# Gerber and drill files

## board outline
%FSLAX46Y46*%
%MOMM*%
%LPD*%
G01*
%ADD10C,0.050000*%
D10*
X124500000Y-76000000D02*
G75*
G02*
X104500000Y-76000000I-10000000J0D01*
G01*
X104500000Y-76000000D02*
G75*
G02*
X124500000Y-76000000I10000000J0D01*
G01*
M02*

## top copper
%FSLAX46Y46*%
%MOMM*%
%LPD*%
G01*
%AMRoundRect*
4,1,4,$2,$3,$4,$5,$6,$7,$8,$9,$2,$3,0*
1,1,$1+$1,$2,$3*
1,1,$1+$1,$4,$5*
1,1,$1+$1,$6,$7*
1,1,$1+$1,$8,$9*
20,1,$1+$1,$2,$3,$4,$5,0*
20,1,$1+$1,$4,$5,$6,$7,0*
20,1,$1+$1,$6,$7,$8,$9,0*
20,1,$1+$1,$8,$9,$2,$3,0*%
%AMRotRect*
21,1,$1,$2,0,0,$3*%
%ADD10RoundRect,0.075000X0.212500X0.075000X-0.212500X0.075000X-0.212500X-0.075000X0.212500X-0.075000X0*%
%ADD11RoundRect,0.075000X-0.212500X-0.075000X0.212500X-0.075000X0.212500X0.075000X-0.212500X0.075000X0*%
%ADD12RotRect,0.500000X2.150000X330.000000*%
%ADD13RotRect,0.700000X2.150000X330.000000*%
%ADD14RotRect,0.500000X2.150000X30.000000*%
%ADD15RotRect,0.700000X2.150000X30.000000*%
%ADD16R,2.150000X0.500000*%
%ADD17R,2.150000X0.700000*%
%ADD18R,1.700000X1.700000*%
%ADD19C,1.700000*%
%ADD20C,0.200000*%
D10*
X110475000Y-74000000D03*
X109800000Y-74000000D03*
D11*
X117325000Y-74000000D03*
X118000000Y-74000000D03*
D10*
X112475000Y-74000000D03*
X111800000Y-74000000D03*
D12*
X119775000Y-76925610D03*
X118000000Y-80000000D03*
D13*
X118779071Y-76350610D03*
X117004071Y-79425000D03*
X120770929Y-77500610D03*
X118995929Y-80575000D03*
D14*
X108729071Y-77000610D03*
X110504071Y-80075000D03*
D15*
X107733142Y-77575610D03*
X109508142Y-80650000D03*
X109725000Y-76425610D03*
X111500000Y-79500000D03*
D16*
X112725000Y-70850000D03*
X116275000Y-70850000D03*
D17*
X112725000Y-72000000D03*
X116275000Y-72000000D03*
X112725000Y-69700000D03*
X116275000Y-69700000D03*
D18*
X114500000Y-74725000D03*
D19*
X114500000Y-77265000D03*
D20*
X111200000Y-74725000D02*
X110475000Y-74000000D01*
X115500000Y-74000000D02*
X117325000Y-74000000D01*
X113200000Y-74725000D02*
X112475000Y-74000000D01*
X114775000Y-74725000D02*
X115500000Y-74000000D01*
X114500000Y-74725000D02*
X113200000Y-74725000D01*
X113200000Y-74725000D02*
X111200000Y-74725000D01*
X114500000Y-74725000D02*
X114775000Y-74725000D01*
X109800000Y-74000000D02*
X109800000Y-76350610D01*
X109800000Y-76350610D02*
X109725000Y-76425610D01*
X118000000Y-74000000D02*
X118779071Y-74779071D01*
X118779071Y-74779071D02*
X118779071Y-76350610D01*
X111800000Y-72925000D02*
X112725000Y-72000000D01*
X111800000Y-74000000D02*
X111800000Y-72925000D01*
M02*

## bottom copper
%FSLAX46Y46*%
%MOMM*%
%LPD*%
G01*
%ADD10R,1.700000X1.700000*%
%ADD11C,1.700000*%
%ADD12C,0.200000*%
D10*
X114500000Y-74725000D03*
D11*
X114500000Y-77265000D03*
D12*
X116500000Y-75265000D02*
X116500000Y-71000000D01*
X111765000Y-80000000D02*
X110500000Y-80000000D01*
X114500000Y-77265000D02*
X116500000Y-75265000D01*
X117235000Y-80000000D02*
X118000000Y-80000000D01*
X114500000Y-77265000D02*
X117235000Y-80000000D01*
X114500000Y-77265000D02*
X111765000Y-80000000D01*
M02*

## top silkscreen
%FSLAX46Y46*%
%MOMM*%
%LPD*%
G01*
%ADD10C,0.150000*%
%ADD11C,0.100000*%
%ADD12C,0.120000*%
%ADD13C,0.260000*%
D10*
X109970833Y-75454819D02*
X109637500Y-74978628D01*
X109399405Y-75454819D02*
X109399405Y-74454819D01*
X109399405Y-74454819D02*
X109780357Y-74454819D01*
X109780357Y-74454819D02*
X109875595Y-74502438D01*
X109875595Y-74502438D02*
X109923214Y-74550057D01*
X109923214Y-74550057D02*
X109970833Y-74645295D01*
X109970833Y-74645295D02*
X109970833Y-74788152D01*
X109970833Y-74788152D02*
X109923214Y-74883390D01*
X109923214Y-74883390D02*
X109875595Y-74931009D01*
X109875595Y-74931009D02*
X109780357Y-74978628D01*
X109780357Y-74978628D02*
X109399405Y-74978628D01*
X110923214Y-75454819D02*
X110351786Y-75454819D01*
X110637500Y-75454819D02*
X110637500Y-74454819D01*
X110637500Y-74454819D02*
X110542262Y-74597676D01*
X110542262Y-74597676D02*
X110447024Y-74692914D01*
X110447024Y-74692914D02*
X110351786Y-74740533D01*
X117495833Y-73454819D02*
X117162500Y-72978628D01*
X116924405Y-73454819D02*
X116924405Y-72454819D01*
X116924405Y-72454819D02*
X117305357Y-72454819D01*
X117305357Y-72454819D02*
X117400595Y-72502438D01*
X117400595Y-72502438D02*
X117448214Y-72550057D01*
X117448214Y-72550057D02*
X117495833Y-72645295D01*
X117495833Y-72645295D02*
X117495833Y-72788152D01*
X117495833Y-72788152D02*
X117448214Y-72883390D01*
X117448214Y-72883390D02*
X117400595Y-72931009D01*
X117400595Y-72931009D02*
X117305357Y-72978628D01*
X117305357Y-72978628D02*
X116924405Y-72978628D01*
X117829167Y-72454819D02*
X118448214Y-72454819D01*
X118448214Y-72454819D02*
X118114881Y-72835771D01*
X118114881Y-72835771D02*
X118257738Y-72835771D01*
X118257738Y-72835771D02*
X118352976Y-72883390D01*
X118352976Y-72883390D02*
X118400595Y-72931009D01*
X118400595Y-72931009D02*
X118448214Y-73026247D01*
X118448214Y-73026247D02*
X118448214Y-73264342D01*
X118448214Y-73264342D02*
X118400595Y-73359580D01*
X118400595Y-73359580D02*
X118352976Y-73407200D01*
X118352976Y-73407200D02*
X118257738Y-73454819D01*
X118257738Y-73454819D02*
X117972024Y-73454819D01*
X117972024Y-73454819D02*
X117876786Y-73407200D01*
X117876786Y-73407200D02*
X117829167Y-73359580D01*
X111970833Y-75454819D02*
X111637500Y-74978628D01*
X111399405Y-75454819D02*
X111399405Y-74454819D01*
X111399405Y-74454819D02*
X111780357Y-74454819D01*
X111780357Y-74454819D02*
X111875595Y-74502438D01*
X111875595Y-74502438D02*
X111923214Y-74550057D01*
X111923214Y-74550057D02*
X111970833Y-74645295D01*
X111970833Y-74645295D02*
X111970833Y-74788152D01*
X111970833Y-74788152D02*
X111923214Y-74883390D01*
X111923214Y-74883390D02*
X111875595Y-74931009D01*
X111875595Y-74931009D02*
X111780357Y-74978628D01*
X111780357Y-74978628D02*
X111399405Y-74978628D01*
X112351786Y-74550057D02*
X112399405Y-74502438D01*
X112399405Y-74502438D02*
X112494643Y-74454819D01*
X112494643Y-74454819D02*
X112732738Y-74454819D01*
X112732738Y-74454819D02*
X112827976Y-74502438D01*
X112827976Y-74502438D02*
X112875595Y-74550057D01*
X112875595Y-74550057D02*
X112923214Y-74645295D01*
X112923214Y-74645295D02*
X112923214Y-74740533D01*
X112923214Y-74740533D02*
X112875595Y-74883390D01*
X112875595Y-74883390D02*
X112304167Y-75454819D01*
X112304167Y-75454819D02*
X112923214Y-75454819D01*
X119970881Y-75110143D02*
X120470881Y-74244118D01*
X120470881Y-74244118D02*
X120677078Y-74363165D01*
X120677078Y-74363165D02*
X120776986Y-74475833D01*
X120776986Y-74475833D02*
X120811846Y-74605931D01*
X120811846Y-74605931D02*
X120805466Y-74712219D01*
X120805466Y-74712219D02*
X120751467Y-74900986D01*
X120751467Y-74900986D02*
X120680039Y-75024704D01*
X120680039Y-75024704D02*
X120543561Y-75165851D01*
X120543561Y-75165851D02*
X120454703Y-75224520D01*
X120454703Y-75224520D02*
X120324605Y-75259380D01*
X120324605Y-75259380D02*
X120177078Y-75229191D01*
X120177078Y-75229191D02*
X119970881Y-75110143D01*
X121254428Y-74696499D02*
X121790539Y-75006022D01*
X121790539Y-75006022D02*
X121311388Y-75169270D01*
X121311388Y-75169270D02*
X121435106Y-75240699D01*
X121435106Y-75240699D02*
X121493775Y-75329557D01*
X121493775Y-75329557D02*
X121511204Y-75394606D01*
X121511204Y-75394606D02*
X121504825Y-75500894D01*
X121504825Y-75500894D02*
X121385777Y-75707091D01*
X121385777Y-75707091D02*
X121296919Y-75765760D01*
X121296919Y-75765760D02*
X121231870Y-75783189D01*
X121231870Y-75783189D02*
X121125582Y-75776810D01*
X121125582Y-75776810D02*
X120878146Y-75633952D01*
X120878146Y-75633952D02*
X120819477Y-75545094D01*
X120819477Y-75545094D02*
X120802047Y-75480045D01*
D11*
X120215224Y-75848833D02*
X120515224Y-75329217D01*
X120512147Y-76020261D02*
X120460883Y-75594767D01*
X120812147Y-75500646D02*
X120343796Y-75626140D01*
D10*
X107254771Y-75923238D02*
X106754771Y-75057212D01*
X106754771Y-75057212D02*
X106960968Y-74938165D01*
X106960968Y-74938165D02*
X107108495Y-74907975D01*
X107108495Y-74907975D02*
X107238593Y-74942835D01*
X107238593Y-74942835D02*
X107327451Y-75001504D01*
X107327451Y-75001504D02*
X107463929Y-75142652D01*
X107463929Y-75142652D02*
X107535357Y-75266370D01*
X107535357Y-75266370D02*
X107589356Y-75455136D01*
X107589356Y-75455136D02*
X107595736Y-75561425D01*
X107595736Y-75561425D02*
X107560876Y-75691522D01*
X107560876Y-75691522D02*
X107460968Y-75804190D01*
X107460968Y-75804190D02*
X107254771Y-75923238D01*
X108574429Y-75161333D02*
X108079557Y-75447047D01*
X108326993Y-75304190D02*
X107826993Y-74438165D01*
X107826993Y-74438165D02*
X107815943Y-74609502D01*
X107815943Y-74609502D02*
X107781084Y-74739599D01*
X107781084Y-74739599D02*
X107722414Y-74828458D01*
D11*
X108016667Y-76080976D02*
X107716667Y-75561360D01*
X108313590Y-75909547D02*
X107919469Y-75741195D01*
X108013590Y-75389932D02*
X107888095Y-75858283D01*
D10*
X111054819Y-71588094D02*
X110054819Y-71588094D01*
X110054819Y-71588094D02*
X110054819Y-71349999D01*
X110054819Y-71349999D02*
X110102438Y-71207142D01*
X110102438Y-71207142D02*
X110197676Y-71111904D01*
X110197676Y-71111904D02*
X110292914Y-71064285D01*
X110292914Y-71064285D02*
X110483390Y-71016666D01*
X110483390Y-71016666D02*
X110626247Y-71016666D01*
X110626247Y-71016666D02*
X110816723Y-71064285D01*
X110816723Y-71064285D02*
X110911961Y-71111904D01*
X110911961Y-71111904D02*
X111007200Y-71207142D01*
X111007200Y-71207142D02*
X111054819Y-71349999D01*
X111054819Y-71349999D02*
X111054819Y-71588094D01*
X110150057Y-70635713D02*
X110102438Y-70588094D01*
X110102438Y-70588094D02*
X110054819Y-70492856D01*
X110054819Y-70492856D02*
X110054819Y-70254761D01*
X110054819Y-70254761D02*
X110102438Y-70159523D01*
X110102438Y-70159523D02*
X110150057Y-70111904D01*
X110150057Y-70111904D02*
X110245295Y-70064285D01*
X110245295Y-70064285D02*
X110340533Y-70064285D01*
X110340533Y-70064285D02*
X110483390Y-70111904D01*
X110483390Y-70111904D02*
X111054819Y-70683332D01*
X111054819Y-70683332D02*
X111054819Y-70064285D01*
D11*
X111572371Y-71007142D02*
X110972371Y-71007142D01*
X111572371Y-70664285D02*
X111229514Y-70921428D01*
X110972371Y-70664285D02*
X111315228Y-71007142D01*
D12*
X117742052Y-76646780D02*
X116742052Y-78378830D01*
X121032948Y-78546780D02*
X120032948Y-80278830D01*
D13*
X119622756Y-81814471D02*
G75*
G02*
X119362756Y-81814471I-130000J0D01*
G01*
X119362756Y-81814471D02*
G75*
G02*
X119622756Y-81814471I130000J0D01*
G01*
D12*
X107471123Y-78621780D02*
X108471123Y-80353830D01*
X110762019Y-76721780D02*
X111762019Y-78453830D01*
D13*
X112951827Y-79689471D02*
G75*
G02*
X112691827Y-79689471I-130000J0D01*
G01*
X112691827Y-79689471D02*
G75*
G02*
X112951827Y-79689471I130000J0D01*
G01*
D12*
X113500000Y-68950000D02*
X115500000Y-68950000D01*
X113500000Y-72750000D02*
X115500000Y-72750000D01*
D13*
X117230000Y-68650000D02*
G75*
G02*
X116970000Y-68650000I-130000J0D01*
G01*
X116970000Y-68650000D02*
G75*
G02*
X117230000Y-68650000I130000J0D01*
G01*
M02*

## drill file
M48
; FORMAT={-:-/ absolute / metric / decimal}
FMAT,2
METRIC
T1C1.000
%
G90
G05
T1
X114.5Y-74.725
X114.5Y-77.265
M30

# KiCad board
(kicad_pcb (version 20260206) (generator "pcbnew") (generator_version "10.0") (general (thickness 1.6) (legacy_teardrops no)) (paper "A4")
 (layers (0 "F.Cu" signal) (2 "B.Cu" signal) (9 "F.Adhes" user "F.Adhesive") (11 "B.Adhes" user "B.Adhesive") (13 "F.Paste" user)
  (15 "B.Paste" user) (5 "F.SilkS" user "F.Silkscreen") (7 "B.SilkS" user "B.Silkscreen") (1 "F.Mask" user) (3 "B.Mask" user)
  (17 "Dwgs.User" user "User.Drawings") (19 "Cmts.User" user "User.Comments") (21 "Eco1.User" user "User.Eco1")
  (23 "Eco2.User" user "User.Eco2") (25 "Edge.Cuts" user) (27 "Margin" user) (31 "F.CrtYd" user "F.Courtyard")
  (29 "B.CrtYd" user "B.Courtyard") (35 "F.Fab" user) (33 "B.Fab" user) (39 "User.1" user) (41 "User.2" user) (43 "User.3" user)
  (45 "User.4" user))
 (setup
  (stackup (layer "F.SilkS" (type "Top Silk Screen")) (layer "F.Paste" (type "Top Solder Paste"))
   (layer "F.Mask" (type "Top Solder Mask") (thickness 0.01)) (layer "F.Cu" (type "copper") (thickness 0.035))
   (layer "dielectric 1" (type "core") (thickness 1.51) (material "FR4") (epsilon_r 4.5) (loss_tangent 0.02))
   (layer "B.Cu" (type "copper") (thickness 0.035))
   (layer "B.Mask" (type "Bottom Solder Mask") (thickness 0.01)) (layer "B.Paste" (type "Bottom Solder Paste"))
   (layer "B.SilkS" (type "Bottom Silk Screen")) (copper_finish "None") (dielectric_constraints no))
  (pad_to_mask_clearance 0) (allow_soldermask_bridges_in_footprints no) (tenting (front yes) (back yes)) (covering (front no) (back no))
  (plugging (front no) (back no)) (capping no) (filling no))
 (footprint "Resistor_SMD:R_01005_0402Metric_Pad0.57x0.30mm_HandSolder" (layer "F.Cu") (at 110.1375 74 180)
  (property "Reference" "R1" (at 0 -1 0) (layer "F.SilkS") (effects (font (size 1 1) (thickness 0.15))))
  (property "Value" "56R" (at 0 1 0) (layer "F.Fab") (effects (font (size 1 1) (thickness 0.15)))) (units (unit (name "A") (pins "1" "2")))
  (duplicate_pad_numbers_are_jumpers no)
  (pad "" smd roundrect (at -0.3625 0 180) (size 0.41 0.27) (layers "F.Paste") (roundrect_rratio 0.25))
  (pad "" smd roundrect (at 0.3625 0 180) (size 0.41 0.27) (layers "F.Paste") (roundrect_rratio 0.25))
  (pad "1" smd roundrect (at -0.3375 0 180) (size 0.575 0.3) (layers "F.Cu" "F.Mask") (roundrect_rratio 0.25) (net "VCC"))
  (pad "2" smd roundrect (at 0.3375 0 180) (size 0.575 0.3) (layers "F.Cu" "F.Mask") (roundrect_rratio 0.25) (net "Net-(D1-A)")))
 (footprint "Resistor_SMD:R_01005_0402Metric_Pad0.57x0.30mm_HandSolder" (layer "F.Cu") (at 117.6625 74)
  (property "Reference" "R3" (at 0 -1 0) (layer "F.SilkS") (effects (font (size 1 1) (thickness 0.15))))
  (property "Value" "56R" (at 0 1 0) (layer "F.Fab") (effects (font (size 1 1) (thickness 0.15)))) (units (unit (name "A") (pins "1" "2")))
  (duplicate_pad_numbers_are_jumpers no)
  (pad "" smd roundrect (at -0.3625 0) (size 0.41 0.27) (layers "F.Paste") (roundrect_rratio 0.25))
  (pad "" smd roundrect (at 0.3625 0) (size 0.41 0.27) (layers "F.Paste") (roundrect_rratio 0.25))
  (pad "1" smd roundrect (at -0.3375 0) (size 0.575 0.3) (layers "F.Cu" "F.Mask") (roundrect_rratio 0.25) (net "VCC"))
  (pad "2" smd roundrect (at 0.3375 0) (size 0.575 0.3) (layers "F.Cu" "F.Mask") (roundrect_rratio 0.25) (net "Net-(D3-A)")))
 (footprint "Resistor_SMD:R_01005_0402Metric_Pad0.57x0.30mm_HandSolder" (layer "F.Cu") (at 112.1375 74 180)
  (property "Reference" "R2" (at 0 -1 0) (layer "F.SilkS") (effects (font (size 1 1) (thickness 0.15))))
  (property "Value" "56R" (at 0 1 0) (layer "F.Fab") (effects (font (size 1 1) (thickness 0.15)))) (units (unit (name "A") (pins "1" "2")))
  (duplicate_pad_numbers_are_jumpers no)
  (pad "" smd roundrect (at -0.3625 0 180) (size 0.41 0.27) (layers "F.Paste") (roundrect_rratio 0.25))
  (pad "" smd roundrect (at 0.3625 0 180) (size 0.41 0.27) (layers "F.Paste") (roundrect_rratio 0.25))
  (pad "1" smd roundrect (at -0.3375 0 180) (size 0.575 0.3) (layers "F.Cu" "F.Mask") (roundrect_rratio 0.25) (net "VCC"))
  (pad "2" smd roundrect (at 0.3375 0 180) (size 0.575 0.3) (layers "F.Cu" "F.Mask") (roundrect_rratio 0.25) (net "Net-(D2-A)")))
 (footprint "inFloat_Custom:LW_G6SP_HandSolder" (layer "F.Cu") (at 118.8875 78.462805 -30)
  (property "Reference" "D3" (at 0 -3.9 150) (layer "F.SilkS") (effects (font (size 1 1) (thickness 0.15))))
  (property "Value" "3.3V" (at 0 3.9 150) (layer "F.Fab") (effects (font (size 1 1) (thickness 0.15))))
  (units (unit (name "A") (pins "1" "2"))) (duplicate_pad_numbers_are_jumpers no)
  (fp_line (start -1.9 -1) (end -1.9 1) (stroke (width 0.12) (type solid)) (layer "F.SilkS"))
  (fp_line (start 1.9 -1) (end 1.9 1) (stroke (width 0.12) (type solid)) (layer "F.SilkS"))
  (fp_circle (center 2.2 2.6) (end 2.4 2.6) (stroke (width 0.12) (type solid)) (fill yes) (layer "F.SilkS"))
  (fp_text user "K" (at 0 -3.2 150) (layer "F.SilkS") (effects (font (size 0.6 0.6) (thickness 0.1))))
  (pad "1" smd rect (at 0 -1.775 330) (size 0.5 2.15) (layers "F.Cu" "F.Mask" "F.Paste") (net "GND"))
  (pad "1" smd rect (at 0 1.775 330) (size 0.5 2.15) (layers "F.Cu" "F.Mask" "F.Paste") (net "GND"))
  (pad "2" smd rect (at -1.15 -1.775 330) (size 0.7 2.15) (layers "F.Cu" "F.Mask" "F.Paste") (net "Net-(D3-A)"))
  (pad "2" smd rect (at -1.15 1.775 330) (size 0.7 2.15) (layers "F.Cu" "F.Mask" "F.Paste") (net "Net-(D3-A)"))
  (pad "2" smd rect (at 1.15 -1.775 330) (size 0.7 2.15) (layers "F.Cu" "F.Mask" "F.Paste") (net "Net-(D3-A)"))
  (pad "2" smd rect (at 1.15 1.775 330) (size 0.7 2.15) (layers "F.Cu" "F.Mask" "F.Paste") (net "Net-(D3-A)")))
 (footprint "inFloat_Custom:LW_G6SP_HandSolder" (layer "F.Cu") (at 109.616571 78.537805 30)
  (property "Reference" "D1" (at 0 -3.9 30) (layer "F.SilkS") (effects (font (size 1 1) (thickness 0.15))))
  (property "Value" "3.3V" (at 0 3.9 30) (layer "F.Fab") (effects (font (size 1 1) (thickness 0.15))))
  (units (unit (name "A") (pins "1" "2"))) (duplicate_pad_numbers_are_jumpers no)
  (fp_line (start -1.9 -1) (end -1.9 1) (stroke (width 0.12) (type solid)) (layer "F.SilkS"))
  (fp_line (start 1.9 -1) (end 1.9 1) (stroke (width 0.12) (type solid)) (layer "F.SilkS"))
  (fp_circle (center 2.2 2.6) (end 2.4 2.6) (stroke (width 0.12) (type solid)) (fill yes) (layer "F.SilkS"))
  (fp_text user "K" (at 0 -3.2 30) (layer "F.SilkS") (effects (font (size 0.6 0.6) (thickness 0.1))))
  (pad "1" smd rect (at 0 -1.775 30) (size 0.5 2.15) (layers "F.Cu" "F.Mask" "F.Paste") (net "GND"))
  (pad "1" smd rect (at 0 1.775 30) (size 0.5 2.15) (layers "F.Cu" "F.Mask" "F.Paste") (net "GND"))
  (pad "2" smd rect (at -1.15 -1.775 30) (size 0.7 2.15) (layers "F.Cu" "F.Mask" "F.Paste") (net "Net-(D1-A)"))
  (pad "2" smd rect (at -1.15 1.775 30) (size 0.7 2.15) (layers "F.Cu" "F.Mask" "F.Paste") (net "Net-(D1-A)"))
  (pad "2" smd rect (at 1.15 -1.775 30) (size 0.7 2.15) (layers "F.Cu" "F.Mask" "F.Paste") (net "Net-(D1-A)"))
  (pad "2" smd rect (at 1.15 1.775 30) (size 0.7 2.15) (layers "F.Cu" "F.Mask" "F.Paste") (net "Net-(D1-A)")))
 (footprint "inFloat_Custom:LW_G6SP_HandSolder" (layer "F.Cu") (at 114.5 70.85 90)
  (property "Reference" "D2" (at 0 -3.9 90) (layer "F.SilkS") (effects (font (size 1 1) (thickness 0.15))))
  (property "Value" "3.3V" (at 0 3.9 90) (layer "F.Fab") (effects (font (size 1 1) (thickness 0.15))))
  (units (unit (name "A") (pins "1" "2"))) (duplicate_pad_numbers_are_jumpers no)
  (fp_line (start 1.9 -1) (end 1.9 1) (stroke (width 0.12) (type solid)) (layer "F.SilkS"))
  (fp_line (start -1.9 -1) (end -1.9 1) (stroke (width 0.12) (type solid)) (layer "F.SilkS"))
  (fp_circle (center 2.2 2.6) (end 2.4 2.6) (stroke (width 0.12) (type solid)) (fill yes) (layer "F.SilkS"))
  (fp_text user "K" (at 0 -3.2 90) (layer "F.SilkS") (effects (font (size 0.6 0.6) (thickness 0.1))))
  (pad "1" smd rect (at 0 -1.775 90) (size 0.5 2.15) (layers "F.Cu" "F.Mask" "F.Paste") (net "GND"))
  (pad "1" smd rect (at 0 1.775 90) (size 0.5 2.15) (layers "F.Cu" "F.Mask" "F.Paste") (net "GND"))
  (pad "2" smd rect (at -1.15 -1.775 90) (size 0.7 2.15) (layers "F.Cu" "F.Mask" "F.Paste") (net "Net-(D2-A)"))
  (pad "2" smd rect (at -1.15 1.775 90) (size 0.7 2.15) (layers "F.Cu" "F.Mask" "F.Paste") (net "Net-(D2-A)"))
  (pad "2" smd rect (at 1.15 -1.775 90) (size 0.7 2.15) (layers "F.Cu" "F.Mask" "F.Paste") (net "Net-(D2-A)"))
  (pad "2" smd rect (at 1.15 1.775 90) (size 0.7 2.15) (layers "F.Cu" "F.Mask" "F.Paste") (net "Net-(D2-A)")))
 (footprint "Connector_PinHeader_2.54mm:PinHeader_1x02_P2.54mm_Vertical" (layer "B.Cu") (at 114.5 74.725 180)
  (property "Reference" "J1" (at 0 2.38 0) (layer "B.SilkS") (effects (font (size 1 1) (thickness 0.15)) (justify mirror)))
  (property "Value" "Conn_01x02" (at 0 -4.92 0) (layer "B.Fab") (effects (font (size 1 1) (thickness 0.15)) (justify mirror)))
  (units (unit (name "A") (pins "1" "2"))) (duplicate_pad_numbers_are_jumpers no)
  (pad "1" thru_hole rect (at 0 0 180) (size 1.7 1.7) (drill 1) (layers "*.Cu" "*.Mask") (remove_unused_layers no) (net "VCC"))
  (pad "2" thru_hole circle (at 0 -2.54 180) (size 1.7 1.7) (drill 1) (layers "*.Cu" "*.Mask") (remove_unused_layers no) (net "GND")))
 (gr_circle (center 114.5 76) (end 124.5 76) (stroke (width 0.05) (type solid)) (fill no) (layer "Edge.Cuts"))
 (segment (start 111.2 74.725) (end 110.475 74) (width 0.2) (layer "F.Cu") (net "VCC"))
 (segment (start 115.5 74) (end 117.325 74) (width 0.2) (layer "F.Cu") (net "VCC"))
 (segment (start 113.2 74.725) (end 112.475 74) (width 0.2) (layer "F.Cu") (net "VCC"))
 (segment (start 114.775 74.725) (end 115.5 74) (width 0.2) (layer "F.Cu") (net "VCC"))
 (segment (start 114.5 74.725) (end 113.2 74.725) (width 0.2) (layer "F.Cu") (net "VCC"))
 (segment (start 113.2 74.725) (end 111.2 74.725) (width 0.2) (layer "F.Cu") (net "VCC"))
 (segment (start 114.5 74.725) (end 114.775 74.725) (width 0.2) (layer "F.Cu") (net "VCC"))
 (segment (start 109.8 74) (end 109.8 76.35061) (width 0.2) (layer "F.Cu") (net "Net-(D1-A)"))
 (segment (start 109.8 76.35061) (end 109.725 76.42561) (width 0.2) (layer "F.Cu") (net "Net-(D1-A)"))
 (segment (start 118 74) (end 118.779071 74.779071) (width 0.2) (layer "F.Cu") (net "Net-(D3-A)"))
 (segment (start 118.779071 74.779071) (end 118.779071 76.35061) (width 0.2) (layer "F.Cu") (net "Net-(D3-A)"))
 (segment (start 111.8 72.925) (end 112.725 72) (width 0.2) (layer "F.Cu") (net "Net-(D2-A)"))
 (segment (start 111.8 74) (end 111.8 72.925) (width 0.2) (layer "F.Cu") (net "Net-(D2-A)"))
 (segment (start 116.5 75.265) (end 116.5 71) (width 0.2) (layer "B.Cu") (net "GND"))
 (segment (start 111.765 80) (end 110.5 80) (width 0.2) (layer "B.Cu") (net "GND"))
 (segment (start 114.5 77.265) (end 116.5 75.265) (width 0.2) (layer "B.Cu") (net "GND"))
 (segment (start 117.235 80) (end 118 80) (width 0.2) (layer "B.Cu") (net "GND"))
 (segment (start 114.5 77.265) (end 117.235 80) (width 0.2) (layer "B.Cu") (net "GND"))
 (segment (start 114.5 77.265) (end 111.765 80) (width 0.2) (layer "B.Cu") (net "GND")))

